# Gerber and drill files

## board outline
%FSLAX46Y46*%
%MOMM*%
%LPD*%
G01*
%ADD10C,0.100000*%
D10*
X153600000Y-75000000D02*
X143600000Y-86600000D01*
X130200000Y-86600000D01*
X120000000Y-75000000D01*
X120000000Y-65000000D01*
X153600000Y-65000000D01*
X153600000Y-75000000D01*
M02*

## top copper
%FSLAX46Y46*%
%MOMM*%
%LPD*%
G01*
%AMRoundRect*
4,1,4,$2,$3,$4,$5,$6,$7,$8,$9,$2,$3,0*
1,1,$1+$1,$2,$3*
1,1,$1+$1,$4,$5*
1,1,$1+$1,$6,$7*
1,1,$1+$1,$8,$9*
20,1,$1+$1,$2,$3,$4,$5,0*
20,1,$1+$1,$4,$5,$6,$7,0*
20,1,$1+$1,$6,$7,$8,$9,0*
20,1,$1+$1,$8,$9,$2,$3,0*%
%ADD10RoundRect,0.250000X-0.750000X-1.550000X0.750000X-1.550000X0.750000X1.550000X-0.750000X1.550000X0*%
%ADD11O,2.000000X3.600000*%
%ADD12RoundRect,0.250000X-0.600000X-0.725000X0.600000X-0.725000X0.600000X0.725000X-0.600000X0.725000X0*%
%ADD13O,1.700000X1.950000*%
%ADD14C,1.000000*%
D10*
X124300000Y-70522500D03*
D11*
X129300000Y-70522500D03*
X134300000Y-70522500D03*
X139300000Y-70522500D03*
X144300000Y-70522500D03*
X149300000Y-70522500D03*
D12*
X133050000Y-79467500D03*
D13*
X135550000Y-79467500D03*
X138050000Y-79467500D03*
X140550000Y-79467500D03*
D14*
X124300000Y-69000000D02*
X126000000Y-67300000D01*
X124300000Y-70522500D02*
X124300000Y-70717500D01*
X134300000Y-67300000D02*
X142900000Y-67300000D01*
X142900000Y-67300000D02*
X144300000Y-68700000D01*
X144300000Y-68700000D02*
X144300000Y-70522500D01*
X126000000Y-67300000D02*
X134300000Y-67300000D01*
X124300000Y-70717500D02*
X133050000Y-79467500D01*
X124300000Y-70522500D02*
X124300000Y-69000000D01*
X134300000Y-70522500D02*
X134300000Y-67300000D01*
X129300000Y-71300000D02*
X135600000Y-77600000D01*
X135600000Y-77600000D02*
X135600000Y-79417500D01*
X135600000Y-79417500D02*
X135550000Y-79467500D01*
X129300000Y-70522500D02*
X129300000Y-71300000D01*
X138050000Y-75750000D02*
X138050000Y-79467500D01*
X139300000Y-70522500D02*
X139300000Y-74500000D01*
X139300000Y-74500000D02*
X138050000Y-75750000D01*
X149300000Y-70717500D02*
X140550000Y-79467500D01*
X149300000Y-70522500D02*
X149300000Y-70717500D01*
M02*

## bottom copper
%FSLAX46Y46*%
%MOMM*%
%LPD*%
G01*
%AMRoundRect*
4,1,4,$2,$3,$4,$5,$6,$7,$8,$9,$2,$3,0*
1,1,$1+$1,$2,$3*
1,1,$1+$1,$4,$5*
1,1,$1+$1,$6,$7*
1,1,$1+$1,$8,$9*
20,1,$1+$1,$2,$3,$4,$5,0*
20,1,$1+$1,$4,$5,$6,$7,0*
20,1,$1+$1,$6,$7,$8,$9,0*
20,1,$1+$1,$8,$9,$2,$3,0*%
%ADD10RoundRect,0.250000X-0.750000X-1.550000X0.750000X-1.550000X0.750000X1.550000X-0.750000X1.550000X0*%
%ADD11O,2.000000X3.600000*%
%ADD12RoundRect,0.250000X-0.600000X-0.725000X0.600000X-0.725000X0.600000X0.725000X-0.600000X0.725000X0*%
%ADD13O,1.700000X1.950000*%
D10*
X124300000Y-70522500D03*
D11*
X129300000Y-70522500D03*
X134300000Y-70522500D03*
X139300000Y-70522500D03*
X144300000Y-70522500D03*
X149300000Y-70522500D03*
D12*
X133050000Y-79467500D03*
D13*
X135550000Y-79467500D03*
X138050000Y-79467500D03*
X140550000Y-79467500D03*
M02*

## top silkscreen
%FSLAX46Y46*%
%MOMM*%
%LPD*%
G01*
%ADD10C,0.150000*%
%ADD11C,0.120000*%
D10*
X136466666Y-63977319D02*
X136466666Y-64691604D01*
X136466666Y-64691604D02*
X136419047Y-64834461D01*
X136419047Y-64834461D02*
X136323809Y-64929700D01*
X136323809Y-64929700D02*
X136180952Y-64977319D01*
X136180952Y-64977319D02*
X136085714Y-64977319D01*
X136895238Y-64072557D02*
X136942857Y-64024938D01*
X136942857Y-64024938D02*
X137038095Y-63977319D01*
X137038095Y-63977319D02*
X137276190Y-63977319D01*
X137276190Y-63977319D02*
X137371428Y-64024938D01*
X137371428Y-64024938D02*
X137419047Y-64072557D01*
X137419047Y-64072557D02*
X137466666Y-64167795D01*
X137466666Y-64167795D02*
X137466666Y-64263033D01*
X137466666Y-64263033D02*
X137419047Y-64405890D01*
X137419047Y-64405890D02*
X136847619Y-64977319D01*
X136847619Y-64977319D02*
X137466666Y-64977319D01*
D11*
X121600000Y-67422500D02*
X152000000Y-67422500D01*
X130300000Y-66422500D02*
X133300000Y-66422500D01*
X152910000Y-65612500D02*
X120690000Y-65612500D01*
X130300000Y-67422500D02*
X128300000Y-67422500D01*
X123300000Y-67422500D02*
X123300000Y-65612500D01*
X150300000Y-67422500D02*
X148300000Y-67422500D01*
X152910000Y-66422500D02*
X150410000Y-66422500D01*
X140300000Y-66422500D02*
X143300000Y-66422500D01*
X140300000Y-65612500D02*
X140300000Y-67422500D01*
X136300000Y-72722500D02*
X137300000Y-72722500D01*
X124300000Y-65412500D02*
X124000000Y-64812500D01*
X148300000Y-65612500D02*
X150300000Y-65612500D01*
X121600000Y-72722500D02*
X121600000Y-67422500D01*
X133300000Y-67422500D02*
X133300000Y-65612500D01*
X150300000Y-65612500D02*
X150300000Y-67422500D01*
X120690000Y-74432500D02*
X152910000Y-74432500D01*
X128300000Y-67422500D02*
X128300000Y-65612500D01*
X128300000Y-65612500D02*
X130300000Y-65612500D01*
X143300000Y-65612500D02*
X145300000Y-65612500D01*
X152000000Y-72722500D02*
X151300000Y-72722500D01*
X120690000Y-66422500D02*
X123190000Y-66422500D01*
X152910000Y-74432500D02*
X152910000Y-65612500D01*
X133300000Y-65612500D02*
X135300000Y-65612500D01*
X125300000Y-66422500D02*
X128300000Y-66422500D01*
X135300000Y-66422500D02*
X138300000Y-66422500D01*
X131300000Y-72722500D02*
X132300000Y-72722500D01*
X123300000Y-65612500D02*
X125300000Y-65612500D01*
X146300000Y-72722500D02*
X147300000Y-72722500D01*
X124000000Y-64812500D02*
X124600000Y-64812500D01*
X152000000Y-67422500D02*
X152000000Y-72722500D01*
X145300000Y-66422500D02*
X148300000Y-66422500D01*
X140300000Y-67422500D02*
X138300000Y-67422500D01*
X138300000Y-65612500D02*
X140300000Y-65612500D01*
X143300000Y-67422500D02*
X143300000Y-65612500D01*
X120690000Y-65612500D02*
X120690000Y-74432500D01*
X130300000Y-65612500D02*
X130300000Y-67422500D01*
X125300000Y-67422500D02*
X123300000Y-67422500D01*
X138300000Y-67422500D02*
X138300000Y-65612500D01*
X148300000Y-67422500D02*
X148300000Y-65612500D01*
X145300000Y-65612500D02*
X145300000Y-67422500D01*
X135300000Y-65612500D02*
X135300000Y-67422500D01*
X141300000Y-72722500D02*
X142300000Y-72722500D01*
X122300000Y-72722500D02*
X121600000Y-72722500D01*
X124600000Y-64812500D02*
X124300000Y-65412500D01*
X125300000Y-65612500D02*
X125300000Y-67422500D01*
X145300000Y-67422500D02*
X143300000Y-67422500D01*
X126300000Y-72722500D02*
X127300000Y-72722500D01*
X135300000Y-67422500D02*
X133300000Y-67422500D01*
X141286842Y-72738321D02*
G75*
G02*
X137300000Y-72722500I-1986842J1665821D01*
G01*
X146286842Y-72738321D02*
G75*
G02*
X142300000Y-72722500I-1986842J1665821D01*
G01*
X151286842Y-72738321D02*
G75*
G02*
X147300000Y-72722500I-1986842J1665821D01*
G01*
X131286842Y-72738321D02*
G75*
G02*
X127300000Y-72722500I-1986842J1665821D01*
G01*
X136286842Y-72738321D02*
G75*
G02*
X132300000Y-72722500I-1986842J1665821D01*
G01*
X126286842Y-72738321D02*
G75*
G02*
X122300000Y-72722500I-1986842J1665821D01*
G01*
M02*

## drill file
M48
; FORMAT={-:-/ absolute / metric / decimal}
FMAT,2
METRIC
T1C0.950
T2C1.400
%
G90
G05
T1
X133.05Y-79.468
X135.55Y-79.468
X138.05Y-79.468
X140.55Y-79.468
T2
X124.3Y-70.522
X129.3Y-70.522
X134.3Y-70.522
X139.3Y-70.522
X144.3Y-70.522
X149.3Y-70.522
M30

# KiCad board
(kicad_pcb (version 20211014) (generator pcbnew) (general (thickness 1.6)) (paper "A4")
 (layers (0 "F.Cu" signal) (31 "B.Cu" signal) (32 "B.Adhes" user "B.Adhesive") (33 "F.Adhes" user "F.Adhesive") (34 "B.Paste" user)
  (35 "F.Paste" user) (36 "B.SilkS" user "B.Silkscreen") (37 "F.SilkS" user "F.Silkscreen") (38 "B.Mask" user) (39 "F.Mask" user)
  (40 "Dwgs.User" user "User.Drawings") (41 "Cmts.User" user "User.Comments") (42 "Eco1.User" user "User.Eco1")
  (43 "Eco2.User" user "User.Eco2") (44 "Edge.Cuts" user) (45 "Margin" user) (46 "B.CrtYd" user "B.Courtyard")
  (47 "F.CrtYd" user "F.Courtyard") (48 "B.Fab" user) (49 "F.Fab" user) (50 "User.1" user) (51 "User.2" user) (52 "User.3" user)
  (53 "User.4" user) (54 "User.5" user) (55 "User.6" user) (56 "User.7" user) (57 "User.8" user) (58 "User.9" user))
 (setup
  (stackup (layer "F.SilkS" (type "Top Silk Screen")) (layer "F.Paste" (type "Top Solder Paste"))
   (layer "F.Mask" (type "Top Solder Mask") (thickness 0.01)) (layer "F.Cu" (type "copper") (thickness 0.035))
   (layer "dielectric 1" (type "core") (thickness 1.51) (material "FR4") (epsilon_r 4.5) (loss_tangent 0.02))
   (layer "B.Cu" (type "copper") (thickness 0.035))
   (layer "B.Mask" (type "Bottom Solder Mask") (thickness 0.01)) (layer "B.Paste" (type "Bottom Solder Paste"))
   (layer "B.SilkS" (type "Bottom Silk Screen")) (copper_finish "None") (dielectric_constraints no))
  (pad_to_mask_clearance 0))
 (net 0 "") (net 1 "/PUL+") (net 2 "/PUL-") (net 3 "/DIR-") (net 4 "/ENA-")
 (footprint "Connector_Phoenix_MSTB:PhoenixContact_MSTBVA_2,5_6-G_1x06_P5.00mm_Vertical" (layer "F.Cu") (at 124.3 70.5225)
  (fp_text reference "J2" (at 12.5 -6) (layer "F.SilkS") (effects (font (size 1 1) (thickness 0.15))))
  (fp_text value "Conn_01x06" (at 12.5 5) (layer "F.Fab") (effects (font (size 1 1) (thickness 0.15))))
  (fp_line (start -2.7 -3.1) (end 27.7 -3.1) (layer "F.SilkS") (width 0.12))
  (fp_line (start 6 -4.1) (end 9 -4.1) (layer "F.SilkS") (width 0.12))
  (fp_line (start 28.61 -4.91) (end -3.61 -4.91) (layer "F.SilkS") (width 0.12))
  (fp_line (start 6 -3.1) (end 4 -3.1) (layer "F.SilkS") (width 0.12))
  (fp_line (start -1 -3.1) (end -1 -4.91) (layer "F.SilkS") (width 0.12))
  (fp_line (start 26 -3.1) (end 24 -3.1) (layer "F.SilkS") (width 0.12))
  (fp_line (start 28.61 -4.1) (end 26.11 -4.1) (layer "F.SilkS") (width 0.12))
  (fp_line (start 16 -4.1) (end 19 -4.1) (layer "F.SilkS") (width 0.12))
  (fp_line (start 16 -4.91) (end 16 -3.1) (layer "F.SilkS") (width 0.12))
  (fp_line (start 12 2.2) (end 13 2.2) (layer "F.SilkS") (width 0.12))
  (fp_line (start 0 -5.11) (end -0.3 -5.71) (layer "F.SilkS") (width 0.12))
  (fp_line (start 24 -4.91) (end 26 -4.91) (layer "F.SilkS") (width 0.12))
  (fp_line (start -2.7 2.2) (end -2.7 -3.1) (layer "F.SilkS") (width 0.12))
  (fp_line (start 9 -3.1) (end 9 -4.91) (layer "F.SilkS") (width 0.12))
  (fp_line (start 26 -4.91) (end 26 -3.1) (layer "F.SilkS") (width 0.12))
  (fp_line (start -3.61 3.91) (end 28.61 3.91) (layer "F.SilkS") (width 0.12))
  (fp_line (start 4 -3.1) (end 4 -4.91) (layer "F.SilkS") (width 0.12))
  (fp_line (start 4 -4.91) (end 6 -4.91) (layer "F.SilkS") (width 0.12))
  (fp_line (start 19 -4.91) (end 21 -4.91) (layer "F.SilkS") (width 0.12))
  (fp_line (start 27.7 2.2) (end 27 2.2) (layer "F.SilkS") (width 0.12))
  (fp_line (start -3.61 -4.1) (end -1.11 -4.1) (layer "F.SilkS") (width 0.12))
  (fp_line (start 28.61 3.91) (end 28.61 -4.91) (layer "F.SilkS") (width 0.12))
  (fp_line (start 9 -4.91) (end 11 -4.91) (layer "F.SilkS") (width 0.12))
  (fp_line (start 1 -4.1) (end 4 -4.1) (layer "F.SilkS") (width 0.12))
  (fp_line (start 11 -4.1) (end 14 -4.1) (layer "F.SilkS") (width 0.12))
  (fp_line (start 7 2.2) (end 8 2.2) (layer "F.SilkS") (width 0.12))
  (fp_line (start -1 -4.91) (end 1 -4.91) (layer "F.SilkS") (width 0.12))
  (fp_line (start 22 2.2) (end 23 2.2) (layer "F.SilkS") (width 0.12))
  (fp_line (start -0.3 -5.71) (end 0.3 -5.71) (layer "F.SilkS") (width 0.12))
  (fp_line (start 27.7 -3.1) (end 27.7 2.2) (layer "F.SilkS") (width 0.12))
  (fp_line (start 21 -4.1) (end 24 -4.1) (layer "F.SilkS") (width 0.12))
  (fp_line (start 16 -3.1) (end 14 -3.1) (layer "F.SilkS") (width 0.12))
  (fp_line (start 14 -4.91) (end 16 -4.91) (layer "F.SilkS") (width 0.12))
  (fp_line (start 19 -3.1) (end 19 -4.91) (layer "F.SilkS") (width 0.12))
  (fp_line (start -3.61 -4.91) (end -3.61 3.91) (layer "F.SilkS") (width 0.12))
  (fp_line (start 6 -4.91) (end 6 -3.1) (layer "F.SilkS") (width 0.12))
  (fp_line (start 1 -3.1) (end -1 -3.1) (layer "F.SilkS") (width 0.12))
  (fp_line (start 14 -3.1) (end 14 -4.91) (layer "F.SilkS") (width 0.12))
  (fp_line (start 24 -3.1) (end 24 -4.91) (layer "F.SilkS") (width 0.12))
  (fp_line (start 21 -4.91) (end 21 -3.1) (layer "F.SilkS") (width 0.12))
  (fp_line (start 11 -4.91) (end 11 -3.1) (layer "F.SilkS") (width 0.12))
  (fp_line (start 17 2.2) (end 18 2.2) (layer "F.SilkS") (width 0.12))
  (fp_line (start -2 2.2) (end -2.7 2.2) (layer "F.SilkS") (width 0.12))
  (fp_line (start 0.3 -5.71) (end 0 -5.11) (layer "F.SilkS") (width 0.12))
  (fp_line (start 1 -4.91) (end 1 -3.1) (layer "F.SilkS") (width 0.12))
  (fp_line (start 21 -3.1) (end 19 -3.1) (layer "F.SilkS") (width 0.12))
  (fp_line (start 2 2.2) (end 3 2.2) (layer "F.SilkS") (width 0.12))
  (fp_line (start 11 -3.1) (end 9 -3.1) (layer "F.SilkS") (width 0.12))
  (fp_arc (start 16.986842 2.215821) (mid 14.989711 3.142758) (end 13 2.2) (layer "F.SilkS") (width 0.12))
  (fp_arc (start 21.986842 2.215821) (mid 19.989711 3.142758) (end 18 2.2) (layer "F.SilkS") (width 0.12))
  (fp_arc (start 26.986842 2.215821) (mid 24.989711 3.142758) (end 23 2.2) (layer "F.SilkS") (width 0.12))
  (fp_arc (start 6.986842 2.215821) (mid 4.989711 3.142758) (end 3 2.2) (layer "F.SilkS") (width 0.12))
  (fp_arc (start 11.986842 2.215821) (mid 9.989711 3.142758) (end 8 2.2) (layer "F.SilkS") (width 0.12))
  (fp_arc (start 1.986842 2.215821) (mid -0.010289 3.142758) (end -2 2.2) (layer "F.SilkS") (width 0.12))
  (pad "1" thru_hole roundrect (at 0 0) (size 2 3.6) (drill 1.4) (layers *.Cu *.Mask) (roundrect_rratio 0.125) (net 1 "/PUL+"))
  (pad "2" thru_hole oval (at 5 0) (size 2 3.6) (drill 1.4) (layers *.Cu *.Mask) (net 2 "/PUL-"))
  (pad "3" thru_hole oval (at 10 0) (size 2 3.6) (drill 1.4) (layers *.Cu *.Mask) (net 1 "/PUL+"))
  (pad "4" thru_hole oval (at 15 0) (size 2 3.6) (drill 1.4) (layers *.Cu *.Mask) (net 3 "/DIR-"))
  (pad "5" thru_hole oval (at 20 0) (size 2 3.6) (drill 1.4) (layers *.Cu *.Mask) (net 1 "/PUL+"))
  (pad "6" thru_hole oval (at 25 0) (size 2 3.6) (drill 1.4) (layers *.Cu *.Mask) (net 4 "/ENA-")))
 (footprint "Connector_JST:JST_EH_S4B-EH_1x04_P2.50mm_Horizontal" (layer "B.Cu") (at 133.05 79.4675)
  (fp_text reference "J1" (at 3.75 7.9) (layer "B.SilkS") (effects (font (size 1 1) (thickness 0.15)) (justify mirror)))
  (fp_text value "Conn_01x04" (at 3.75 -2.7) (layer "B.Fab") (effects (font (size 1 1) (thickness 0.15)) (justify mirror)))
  (pad "1" thru_hole roundrect (at 0 0) (size 1.7 1.95) (drill 0.95) (layers *.Cu *.Mask) (roundrect_rratio 0.147059) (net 1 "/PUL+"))
  (pad "2" thru_hole oval (at 2.5 0) (size 1.7 1.95) (drill 0.95) (layers *.Cu *.Mask) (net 2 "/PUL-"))
  (pad "3" thru_hole oval (at 5 0) (size 1.7 1.95) (drill 0.95) (layers *.Cu *.Mask) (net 3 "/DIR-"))
  (pad "4" thru_hole oval (at 7.5 0) (size 1.7 1.95) (drill 0.95) (layers *.Cu *.Mask) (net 4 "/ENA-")))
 (gr_poly
  (pts (xy 153.6 75) (xy 143.6 86.6) (xy 130.2 86.6) (xy 120 75) (xy 120 65) (xy 153.6 65)) (layer "Edge.Cuts") (width 0.1) (fill none))
 (segment (start 124.3 69) (end 126 67.3) (width 1) (layer "F.Cu") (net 1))
 (segment (start 124.3 70.5225) (end 124.3 70.7175) (width 1) (layer "F.Cu") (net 1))
 (segment (start 134.3 67.3) (end 142.9 67.3) (width 1) (layer "F.Cu") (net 1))
 (segment (start 142.9 67.3) (end 144.3 68.7) (width 1) (layer "F.Cu") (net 1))
 (segment (start 144.3 68.7) (end 144.3 70.5225) (width 1) (layer "F.Cu") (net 1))
 (segment (start 126 67.3) (end 134.3 67.3) (width 1) (layer "F.Cu") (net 1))
 (segment (start 124.3 70.7175) (end 133.05 79.4675) (width 1) (layer "F.Cu") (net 1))
 (segment (start 124.3 70.5225) (end 124.3 69) (width 1) (layer "F.Cu") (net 1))
 (segment (start 134.3 70.5225) (end 134.3 67.3) (width 1) (layer "F.Cu") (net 1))
 (segment (start 129.3 71.3) (end 135.6 77.6) (width 1) (layer "F.Cu") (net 2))
 (segment (start 135.6 77.6) (end 135.6 79.4175) (width 1) (layer "F.Cu") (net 2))
 (segment (start 135.6 79.4175) (end 135.55 79.4675) (width 1) (layer "F.Cu") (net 2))
 (segment (start 129.3 70.5225) (end 129.3 71.3) (width 1) (layer "F.Cu") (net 2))
 (segment (start 138.05 75.75) (end 138.05 79.4675) (width 1) (layer "F.Cu") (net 3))
 (segment (start 139.3 70.5225) (end 139.3 74.5) (width 1) (layer "F.Cu") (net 3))
 (segment (start 139.3 74.5) (end 138.05 75.75) (width 1) (layer "F.Cu") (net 3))
 (segment (start 149.3 70.7175) (end 140.55 79.4675) (width 1) (layer "F.Cu") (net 4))
 (segment (start 149.3 70.5225) (end 149.3 70.7175) (width 1) (layer "F.Cu") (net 4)))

